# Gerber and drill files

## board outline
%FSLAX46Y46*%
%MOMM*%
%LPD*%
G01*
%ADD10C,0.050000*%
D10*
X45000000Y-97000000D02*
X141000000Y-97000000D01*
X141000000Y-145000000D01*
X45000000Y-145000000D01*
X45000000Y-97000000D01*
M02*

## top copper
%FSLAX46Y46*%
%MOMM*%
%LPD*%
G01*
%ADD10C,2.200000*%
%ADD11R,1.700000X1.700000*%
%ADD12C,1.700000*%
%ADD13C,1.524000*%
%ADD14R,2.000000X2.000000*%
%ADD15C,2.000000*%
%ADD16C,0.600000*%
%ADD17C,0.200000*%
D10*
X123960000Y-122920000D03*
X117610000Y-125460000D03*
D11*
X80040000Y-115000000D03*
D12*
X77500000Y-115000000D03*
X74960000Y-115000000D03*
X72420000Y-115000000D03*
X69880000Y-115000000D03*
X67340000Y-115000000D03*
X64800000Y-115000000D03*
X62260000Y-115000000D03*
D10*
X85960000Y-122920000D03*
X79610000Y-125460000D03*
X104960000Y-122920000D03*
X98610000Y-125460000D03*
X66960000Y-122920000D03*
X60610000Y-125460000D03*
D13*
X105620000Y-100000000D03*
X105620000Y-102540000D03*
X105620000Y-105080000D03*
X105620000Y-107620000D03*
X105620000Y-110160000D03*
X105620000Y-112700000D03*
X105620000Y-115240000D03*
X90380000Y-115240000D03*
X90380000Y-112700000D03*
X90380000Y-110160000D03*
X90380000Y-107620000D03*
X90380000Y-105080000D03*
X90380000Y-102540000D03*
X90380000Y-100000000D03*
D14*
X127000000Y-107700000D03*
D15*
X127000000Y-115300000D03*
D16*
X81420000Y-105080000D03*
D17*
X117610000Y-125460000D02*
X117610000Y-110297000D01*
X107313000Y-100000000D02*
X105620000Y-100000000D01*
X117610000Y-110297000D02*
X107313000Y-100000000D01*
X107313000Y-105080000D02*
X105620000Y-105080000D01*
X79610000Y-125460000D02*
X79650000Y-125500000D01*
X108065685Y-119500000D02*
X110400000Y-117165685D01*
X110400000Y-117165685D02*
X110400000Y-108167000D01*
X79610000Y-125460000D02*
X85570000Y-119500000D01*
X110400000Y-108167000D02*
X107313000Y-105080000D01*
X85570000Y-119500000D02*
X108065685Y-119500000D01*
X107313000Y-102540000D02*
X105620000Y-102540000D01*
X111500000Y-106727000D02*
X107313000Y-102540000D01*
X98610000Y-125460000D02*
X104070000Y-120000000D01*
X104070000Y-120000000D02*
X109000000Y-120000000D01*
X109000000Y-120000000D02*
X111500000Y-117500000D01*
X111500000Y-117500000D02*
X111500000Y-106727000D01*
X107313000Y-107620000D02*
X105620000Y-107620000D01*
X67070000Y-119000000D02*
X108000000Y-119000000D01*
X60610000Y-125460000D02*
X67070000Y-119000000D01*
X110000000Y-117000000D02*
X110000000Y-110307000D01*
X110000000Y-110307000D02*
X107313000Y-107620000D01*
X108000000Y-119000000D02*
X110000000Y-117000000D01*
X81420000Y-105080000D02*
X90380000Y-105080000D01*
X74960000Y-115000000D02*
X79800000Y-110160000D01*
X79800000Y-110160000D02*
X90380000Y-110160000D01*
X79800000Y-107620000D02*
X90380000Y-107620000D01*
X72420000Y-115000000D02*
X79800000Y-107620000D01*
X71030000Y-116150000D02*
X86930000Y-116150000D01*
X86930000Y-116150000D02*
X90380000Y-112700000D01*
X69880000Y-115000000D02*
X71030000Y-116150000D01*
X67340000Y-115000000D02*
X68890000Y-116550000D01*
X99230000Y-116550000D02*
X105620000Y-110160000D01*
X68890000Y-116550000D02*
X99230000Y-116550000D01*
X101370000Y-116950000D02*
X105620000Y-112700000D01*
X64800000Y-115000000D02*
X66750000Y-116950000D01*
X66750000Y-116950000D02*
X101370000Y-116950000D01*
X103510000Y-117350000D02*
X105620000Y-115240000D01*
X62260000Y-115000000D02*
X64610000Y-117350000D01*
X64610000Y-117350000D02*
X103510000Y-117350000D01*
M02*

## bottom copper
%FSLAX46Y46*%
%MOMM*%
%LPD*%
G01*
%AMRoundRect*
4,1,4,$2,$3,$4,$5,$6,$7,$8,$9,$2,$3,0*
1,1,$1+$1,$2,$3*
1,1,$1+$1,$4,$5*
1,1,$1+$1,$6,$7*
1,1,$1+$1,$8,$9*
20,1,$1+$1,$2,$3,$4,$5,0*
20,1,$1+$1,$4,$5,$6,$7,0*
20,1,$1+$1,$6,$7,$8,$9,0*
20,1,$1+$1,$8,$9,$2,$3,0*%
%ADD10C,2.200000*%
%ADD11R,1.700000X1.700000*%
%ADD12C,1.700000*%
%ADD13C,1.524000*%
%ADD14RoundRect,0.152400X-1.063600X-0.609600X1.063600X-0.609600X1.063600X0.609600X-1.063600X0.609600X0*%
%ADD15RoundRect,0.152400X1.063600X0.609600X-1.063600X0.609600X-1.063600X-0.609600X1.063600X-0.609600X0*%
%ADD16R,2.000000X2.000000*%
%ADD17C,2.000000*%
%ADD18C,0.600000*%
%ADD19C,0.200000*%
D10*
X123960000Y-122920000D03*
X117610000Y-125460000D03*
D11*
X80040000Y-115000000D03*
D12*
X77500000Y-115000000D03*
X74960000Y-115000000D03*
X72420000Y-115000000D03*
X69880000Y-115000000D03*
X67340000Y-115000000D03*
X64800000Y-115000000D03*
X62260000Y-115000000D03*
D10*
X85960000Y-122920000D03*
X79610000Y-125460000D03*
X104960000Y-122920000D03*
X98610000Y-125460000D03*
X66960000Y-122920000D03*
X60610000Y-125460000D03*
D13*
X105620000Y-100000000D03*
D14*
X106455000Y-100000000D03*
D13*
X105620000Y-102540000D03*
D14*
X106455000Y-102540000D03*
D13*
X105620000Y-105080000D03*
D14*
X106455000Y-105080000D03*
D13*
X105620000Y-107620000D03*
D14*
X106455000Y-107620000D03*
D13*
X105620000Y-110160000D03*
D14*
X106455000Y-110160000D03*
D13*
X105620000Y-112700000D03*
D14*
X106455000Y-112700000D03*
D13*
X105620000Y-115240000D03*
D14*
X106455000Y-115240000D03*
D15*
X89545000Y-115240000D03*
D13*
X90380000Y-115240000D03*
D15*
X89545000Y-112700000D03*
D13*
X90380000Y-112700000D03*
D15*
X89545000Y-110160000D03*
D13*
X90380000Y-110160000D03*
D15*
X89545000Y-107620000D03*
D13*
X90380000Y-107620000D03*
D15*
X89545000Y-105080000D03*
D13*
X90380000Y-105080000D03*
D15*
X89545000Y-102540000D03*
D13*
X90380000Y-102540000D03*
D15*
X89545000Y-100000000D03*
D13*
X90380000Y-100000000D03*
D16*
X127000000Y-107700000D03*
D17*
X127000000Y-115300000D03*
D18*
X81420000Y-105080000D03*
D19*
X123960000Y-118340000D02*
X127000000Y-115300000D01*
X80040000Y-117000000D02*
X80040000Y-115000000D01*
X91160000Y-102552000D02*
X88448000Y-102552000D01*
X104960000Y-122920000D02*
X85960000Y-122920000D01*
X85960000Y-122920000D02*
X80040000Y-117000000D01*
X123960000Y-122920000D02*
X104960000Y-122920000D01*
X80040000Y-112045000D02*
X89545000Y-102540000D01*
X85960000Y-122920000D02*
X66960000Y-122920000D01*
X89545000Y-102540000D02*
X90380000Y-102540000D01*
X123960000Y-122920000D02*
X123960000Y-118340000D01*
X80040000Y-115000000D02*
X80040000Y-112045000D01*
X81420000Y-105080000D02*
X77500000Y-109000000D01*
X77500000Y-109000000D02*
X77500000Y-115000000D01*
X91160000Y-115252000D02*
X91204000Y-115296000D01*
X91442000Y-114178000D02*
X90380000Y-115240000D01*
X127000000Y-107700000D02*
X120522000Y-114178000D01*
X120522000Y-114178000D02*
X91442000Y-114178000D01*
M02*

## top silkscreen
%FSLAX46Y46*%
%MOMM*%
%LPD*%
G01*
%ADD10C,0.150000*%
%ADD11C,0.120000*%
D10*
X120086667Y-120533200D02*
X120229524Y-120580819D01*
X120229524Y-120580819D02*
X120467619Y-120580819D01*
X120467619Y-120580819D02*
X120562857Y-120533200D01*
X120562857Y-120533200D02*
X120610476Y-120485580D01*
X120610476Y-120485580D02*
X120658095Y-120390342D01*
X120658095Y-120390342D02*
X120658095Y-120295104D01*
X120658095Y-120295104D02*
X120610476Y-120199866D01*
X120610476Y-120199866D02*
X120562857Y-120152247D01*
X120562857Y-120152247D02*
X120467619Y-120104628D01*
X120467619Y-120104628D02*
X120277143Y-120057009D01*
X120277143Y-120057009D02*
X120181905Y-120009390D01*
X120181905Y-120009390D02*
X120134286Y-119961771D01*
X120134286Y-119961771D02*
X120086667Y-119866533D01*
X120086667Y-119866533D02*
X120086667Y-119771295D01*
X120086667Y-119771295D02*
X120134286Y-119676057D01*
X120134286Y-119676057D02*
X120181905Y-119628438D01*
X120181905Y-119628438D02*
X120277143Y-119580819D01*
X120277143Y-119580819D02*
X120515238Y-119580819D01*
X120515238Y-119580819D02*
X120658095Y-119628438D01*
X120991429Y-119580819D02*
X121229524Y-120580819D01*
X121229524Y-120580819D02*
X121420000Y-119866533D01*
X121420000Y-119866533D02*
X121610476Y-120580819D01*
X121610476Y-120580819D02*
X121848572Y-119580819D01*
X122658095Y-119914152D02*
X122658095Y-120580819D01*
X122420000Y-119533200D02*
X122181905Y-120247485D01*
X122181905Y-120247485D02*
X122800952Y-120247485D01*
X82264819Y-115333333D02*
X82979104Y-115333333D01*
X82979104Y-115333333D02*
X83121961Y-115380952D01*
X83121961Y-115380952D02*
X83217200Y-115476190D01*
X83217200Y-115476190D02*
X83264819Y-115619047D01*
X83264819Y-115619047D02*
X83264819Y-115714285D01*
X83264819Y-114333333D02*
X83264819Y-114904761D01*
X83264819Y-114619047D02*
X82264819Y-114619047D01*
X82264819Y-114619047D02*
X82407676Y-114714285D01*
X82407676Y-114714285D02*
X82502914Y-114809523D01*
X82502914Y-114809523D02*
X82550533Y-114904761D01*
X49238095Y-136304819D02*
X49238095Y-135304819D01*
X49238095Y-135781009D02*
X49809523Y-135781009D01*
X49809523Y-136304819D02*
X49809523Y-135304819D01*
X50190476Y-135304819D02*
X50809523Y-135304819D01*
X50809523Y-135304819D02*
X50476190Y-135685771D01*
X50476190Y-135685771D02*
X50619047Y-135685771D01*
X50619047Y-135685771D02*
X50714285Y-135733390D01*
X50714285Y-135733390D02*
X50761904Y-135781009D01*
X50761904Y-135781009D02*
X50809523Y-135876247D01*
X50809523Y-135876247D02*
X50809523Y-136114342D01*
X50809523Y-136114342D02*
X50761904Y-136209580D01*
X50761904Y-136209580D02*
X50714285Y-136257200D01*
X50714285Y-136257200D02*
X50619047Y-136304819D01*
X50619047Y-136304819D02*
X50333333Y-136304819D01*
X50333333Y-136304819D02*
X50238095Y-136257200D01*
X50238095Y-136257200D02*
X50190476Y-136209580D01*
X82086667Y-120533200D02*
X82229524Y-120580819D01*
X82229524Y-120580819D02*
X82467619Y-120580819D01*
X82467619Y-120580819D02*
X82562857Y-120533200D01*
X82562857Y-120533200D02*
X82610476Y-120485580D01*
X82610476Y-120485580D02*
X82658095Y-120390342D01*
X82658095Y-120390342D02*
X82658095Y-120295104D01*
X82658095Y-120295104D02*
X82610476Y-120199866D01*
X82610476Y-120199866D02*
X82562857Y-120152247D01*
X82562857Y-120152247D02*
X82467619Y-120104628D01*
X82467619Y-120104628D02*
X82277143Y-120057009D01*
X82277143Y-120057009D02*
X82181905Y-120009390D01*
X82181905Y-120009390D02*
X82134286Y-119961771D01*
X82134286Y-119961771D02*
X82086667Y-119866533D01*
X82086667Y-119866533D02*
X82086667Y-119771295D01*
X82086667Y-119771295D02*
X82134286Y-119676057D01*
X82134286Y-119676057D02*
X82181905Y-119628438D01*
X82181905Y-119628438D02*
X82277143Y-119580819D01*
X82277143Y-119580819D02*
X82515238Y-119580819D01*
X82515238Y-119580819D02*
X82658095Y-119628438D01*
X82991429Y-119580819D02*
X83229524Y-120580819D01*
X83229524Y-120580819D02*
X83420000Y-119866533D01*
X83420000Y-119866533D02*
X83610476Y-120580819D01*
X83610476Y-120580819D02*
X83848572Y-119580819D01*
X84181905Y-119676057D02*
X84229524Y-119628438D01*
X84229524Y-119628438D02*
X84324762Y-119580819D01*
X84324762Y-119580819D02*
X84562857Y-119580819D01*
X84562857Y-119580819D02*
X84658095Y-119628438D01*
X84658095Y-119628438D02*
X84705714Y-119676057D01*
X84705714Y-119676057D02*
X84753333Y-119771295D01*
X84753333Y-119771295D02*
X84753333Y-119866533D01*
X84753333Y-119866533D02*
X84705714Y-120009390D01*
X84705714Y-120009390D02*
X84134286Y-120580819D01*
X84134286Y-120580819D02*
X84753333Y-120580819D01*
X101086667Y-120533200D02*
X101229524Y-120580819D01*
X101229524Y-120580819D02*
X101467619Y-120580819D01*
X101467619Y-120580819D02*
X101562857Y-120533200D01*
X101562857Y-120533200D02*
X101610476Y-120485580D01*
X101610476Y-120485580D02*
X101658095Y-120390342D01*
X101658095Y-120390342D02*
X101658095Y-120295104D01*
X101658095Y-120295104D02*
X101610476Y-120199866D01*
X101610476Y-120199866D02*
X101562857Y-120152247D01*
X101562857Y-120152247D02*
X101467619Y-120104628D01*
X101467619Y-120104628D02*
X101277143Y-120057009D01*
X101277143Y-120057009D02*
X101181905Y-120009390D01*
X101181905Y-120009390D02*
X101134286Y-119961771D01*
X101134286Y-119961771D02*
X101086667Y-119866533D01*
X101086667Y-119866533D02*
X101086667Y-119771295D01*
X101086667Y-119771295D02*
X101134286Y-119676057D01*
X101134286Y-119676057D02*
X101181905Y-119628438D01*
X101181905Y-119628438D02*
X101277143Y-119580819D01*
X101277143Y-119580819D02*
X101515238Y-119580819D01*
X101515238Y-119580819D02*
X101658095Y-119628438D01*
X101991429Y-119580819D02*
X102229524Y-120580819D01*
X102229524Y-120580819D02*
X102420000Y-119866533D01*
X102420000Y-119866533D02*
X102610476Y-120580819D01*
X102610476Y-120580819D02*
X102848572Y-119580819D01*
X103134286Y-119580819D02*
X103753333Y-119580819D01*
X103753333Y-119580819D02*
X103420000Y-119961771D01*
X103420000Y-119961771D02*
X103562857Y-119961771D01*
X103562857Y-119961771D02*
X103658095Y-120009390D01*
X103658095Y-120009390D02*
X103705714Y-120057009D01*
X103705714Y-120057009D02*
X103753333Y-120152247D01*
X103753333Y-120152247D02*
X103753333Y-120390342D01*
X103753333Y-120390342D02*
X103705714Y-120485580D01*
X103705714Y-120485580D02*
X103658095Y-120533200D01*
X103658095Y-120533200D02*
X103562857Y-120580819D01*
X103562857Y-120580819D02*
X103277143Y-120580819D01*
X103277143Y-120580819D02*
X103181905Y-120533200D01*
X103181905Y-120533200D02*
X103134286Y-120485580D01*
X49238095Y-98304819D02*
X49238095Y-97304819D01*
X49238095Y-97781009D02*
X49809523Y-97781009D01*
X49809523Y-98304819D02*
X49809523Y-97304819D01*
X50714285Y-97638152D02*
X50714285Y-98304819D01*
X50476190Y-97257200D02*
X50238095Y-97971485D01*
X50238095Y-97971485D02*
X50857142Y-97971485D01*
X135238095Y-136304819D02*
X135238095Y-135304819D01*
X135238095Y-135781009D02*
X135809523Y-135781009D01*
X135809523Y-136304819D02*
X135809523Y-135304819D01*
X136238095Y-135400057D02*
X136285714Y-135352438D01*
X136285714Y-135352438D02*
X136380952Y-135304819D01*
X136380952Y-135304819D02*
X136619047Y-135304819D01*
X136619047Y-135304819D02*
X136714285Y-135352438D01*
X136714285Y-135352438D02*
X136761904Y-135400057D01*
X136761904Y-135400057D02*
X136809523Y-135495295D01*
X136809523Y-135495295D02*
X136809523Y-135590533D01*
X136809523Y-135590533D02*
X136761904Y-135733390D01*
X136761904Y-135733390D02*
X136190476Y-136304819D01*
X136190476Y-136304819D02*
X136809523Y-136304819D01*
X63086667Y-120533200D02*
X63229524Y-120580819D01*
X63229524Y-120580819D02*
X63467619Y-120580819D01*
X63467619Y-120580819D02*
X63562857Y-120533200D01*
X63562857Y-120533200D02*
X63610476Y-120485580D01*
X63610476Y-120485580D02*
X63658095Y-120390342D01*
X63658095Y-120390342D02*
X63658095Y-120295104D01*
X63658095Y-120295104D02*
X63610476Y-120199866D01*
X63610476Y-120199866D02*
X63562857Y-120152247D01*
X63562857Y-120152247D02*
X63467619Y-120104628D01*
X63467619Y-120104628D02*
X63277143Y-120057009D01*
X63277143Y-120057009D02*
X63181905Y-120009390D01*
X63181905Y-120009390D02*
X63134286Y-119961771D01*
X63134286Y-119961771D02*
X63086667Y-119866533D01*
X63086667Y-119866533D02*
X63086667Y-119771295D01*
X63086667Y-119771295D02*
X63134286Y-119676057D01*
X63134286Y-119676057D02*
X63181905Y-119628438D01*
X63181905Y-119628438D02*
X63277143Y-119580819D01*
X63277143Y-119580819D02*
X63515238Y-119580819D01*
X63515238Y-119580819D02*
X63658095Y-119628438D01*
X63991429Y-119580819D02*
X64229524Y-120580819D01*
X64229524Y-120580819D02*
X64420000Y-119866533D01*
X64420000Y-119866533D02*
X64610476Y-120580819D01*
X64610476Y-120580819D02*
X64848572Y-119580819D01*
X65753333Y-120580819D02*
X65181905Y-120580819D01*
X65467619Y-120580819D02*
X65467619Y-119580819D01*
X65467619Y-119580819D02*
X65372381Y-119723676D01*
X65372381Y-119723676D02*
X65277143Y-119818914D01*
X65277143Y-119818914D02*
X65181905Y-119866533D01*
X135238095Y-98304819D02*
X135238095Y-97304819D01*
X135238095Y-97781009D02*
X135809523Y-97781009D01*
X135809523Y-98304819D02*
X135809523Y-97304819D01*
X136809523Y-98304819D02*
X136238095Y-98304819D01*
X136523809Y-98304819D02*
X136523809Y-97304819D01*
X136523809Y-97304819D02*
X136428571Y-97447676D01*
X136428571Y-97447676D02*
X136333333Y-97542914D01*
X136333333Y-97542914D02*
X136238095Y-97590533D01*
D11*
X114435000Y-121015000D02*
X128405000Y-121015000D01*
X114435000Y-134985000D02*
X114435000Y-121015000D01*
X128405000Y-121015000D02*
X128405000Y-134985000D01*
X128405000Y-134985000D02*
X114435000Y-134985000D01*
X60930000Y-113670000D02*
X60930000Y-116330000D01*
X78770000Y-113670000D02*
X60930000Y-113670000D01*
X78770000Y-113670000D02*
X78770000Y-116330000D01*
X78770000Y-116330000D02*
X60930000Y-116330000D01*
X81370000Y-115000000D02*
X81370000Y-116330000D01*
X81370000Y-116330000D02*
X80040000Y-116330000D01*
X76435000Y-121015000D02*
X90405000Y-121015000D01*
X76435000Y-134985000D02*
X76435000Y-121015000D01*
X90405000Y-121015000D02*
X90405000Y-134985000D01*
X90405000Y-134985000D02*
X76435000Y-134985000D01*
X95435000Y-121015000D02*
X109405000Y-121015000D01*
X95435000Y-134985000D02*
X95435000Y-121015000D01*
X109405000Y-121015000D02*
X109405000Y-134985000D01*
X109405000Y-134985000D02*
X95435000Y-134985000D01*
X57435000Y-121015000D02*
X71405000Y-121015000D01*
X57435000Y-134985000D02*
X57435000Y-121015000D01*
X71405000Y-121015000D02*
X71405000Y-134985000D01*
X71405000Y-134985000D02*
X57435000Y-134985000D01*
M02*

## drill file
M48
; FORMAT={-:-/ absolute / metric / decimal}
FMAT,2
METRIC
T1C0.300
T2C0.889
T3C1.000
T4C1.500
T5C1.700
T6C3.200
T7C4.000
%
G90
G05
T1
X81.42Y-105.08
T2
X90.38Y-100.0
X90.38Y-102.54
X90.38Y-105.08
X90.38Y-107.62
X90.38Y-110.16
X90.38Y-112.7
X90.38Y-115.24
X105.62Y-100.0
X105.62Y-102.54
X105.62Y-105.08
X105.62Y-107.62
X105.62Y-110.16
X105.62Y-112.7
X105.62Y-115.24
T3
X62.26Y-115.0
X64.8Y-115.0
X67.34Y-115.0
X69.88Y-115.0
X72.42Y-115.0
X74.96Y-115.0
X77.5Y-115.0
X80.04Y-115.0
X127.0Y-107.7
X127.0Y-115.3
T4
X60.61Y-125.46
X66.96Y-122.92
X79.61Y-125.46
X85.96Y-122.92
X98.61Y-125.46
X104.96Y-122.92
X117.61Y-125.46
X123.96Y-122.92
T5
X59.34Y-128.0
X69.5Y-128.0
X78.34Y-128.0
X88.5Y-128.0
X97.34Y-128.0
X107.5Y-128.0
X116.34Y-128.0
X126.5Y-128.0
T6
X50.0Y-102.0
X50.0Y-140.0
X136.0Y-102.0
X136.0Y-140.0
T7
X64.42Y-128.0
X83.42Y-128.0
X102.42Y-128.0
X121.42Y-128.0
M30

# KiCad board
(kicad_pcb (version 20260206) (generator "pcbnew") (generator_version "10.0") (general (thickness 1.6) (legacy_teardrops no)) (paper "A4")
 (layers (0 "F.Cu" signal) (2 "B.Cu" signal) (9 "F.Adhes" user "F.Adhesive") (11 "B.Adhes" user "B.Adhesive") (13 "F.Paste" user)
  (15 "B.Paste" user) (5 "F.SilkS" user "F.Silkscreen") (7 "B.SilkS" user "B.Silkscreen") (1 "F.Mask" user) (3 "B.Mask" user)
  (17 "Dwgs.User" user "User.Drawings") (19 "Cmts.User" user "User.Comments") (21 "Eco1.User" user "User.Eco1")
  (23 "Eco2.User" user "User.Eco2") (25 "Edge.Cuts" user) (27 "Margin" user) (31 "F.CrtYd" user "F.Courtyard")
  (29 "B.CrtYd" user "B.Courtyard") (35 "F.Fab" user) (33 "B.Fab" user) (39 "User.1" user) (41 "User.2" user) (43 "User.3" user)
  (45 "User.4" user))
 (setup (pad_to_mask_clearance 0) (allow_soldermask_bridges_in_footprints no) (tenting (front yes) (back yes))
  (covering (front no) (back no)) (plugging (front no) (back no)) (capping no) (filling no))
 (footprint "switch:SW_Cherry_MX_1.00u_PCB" (layer "F.Cu") (at 123.96 122.92)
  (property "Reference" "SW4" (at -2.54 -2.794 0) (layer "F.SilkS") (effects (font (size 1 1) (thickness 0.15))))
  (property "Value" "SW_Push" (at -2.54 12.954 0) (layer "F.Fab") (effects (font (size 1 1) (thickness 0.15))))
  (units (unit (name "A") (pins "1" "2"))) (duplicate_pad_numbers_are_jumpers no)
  (fp_line (start -9.525 -1.905) (end 4.445 -1.905) (stroke (width 0.12) (type solid)) (layer "F.SilkS"))
  (fp_line (start -9.525 12.065) (end -9.525 -1.905) (stroke (width 0.12) (type solid)) (layer "F.SilkS"))
  (fp_line (start 4.445 -1.905) (end 4.445 12.065) (stroke (width 0.12) (type solid)) (layer "F.SilkS"))
  (fp_line (start 4.445 12.065) (end -9.525 12.065) (stroke (width 0.12) (type solid)) (layer "F.SilkS"))
  (pad "" np_thru_hole circle (at -7.62 5.08) (size 1.7 1.7) (drill 1.7) (layers "*.Cu" "*.Mask"))
  (pad "" np_thru_hole circle (at -2.54 5.08) (size 4 4) (drill 4) (layers "*.Cu" "*.Mask"))
  (pad "" np_thru_hole circle (at 2.54 5.08) (size 1.7 1.7) (drill 1.7) (layers "*.Cu" "*.Mask"))
  (pad "1" thru_hole circle (at 0 0) (size 2.2 2.2) (drill 1.5) (layers "*.Cu" "*.Mask") (remove_unused_layers no) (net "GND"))
  (pad "2" thru_hole circle (at -6.35 2.54) (size 2.2 2.2) (drill 1.5) (layers "*.Cu" "*.Mask") (remove_unused_layers no)
   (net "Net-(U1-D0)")))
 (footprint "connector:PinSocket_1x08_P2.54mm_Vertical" (layer "F.Cu") (at 80.04 115 -90)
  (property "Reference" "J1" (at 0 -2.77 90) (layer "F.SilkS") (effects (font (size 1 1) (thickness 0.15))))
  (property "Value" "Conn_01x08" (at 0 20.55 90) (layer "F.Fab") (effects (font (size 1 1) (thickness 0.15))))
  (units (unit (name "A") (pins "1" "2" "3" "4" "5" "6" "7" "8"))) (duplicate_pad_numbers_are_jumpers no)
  (fp_line (start -1.33 19.11) (end 1.33 19.11) (stroke (width 0.12) (type solid)) (layer "F.SilkS"))
  (fp_line (start -1.33 1.27) (end -1.33 19.11) (stroke (width 0.12) (type solid)) (layer "F.SilkS"))
  (fp_line (start -1.33 1.27) (end 1.33 1.27) (stroke (width 0.12) (type solid)) (layer "F.SilkS"))
  (fp_line (start 1.33 1.27) (end 1.33 19.11) (stroke (width 0.12) (type solid)) (layer "F.SilkS"))
  (fp_line (start 0 -1.33) (end 1.33 -1.33) (stroke (width 0.12) (type solid)) (layer "F.SilkS"))
  (fp_line (start 1.33 -1.33) (end 1.33 0) (stroke (width 0.12) (type solid)) (layer "F.SilkS"))
  (pad "1" thru_hole rect (at 0 0 270) (size 1.7 1.7) (drill 1) (layers "*.Cu" "*.Mask") (remove_unused_layers no) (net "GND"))
  (pad "2" thru_hole circle (at 0 2.54 270) (size 1.7 1.7) (drill 1) (layers "*.Cu" "*.Mask") (remove_unused_layers no) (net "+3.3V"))
  (pad "3" thru_hole circle (at 0 5.08 270) (size 1.7 1.7) (drill 1) (layers "*.Cu" "*.Mask") (remove_unused_layers no) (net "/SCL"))
  (pad "4" thru_hole circle (at 0 7.62 270) (size 1.7 1.7) (drill 1) (layers "*.Cu" "*.Mask") (remove_unused_layers no) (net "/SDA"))
  (pad "5" thru_hole circle (at 0 10.16 270) (size 1.7 1.7) (drill 1) (layers "*.Cu" "*.Mask") (remove_unused_layers no) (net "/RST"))
  (pad "6" thru_hole circle (at 0 12.7 270) (size 1.7 1.7) (drill 1) (layers "*.Cu" "*.Mask") (remove_unused_layers no) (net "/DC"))
  (pad "7" thru_hole circle (at 0 15.24 270) (size 1.7 1.7) (drill 1) (layers "*.Cu" "*.Mask") (remove_unused_layers no) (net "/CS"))
  (pad "8" thru_hole circle (at 0 17.78 270) (size 1.7 1.7) (drill 1) (layers "*.Cu" "*.Mask") (remove_unused_layers no) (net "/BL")))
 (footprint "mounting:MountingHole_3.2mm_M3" (layer "F.Cu") (at 50 140)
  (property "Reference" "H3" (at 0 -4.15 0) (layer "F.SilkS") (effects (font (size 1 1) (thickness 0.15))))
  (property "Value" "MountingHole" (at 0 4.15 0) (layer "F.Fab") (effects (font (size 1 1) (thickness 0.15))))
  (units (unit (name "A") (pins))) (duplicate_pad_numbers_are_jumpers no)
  (pad "" np_thru_hole circle (at 0 0) (size 3.2 3.2) (drill 3.2) (layers "*.Cu" "*.Mask")))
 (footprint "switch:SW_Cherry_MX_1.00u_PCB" (layer "F.Cu") (at 85.96 122.92)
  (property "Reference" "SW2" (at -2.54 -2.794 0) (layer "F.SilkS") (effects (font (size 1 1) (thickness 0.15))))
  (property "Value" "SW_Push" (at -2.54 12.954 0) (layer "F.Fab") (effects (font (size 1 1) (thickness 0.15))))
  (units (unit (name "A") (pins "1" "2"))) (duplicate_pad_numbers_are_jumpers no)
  (fp_line (start -9.525 -1.905) (end 4.445 -1.905) (stroke (width 0.12) (type solid)) (layer "F.SilkS"))
  (fp_line (start -9.525 12.065) (end -9.525 -1.905) (stroke (width 0.12) (type solid)) (layer "F.SilkS"))
  (fp_line (start 4.445 -1.905) (end 4.445 12.065) (stroke (width 0.12) (type solid)) (layer "F.SilkS"))
  (fp_line (start 4.445 12.065) (end -9.525 12.065) (stroke (width 0.12) (type solid)) (layer "F.SilkS"))
  (pad "" np_thru_hole circle (at -7.62 5.08) (size 1.7 1.7) (drill 1.7) (layers "*.Cu" "*.Mask"))
  (pad "" np_thru_hole circle (at -2.54 5.08) (size 4 4) (drill 4) (layers "*.Cu" "*.Mask"))
  (pad "" np_thru_hole circle (at 2.54 5.08) (size 1.7 1.7) (drill 1.7) (layers "*.Cu" "*.Mask"))
  (pad "1" thru_hole circle (at 0 0) (size 2.2 2.2) (drill 1.5) (layers "*.Cu" "*.Mask") (remove_unused_layers no) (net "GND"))
  (pad "2" thru_hole circle (at -6.35 2.54) (size 2.2 2.2) (drill 1.5) (layers "*.Cu" "*.Mask") (remove_unused_layers no)
   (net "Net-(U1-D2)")))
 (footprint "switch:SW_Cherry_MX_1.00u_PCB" (layer "F.Cu") (at 104.96 122.92)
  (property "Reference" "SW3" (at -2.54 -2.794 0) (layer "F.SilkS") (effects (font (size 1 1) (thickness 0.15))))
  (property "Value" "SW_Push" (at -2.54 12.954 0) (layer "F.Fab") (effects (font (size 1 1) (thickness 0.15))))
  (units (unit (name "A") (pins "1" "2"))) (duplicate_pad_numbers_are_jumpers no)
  (fp_line (start -9.525 -1.905) (end 4.445 -1.905) (stroke (width 0.12) (type solid)) (layer "F.SilkS"))
  (fp_line (start -9.525 12.065) (end -9.525 -1.905) (stroke (width 0.12) (type solid)) (layer "F.SilkS"))
  (fp_line (start 4.445 -1.905) (end 4.445 12.065) (stroke (width 0.12) (type solid)) (layer "F.SilkS"))
  (fp_line (start 4.445 12.065) (end -9.525 12.065) (stroke (width 0.12) (type solid)) (layer "F.SilkS"))
  (pad "" np_thru_hole circle (at -7.62 5.08) (size 1.7 1.7) (drill 1.7) (layers "*.Cu" "*.Mask"))
  (pad "" np_thru_hole circle (at -2.54 5.08) (size 4 4) (drill 4) (layers "*.Cu" "*.Mask"))
  (pad "" np_thru_hole circle (at 2.54 5.08) (size 1.7 1.7) (drill 1.7) (layers "*.Cu" "*.Mask"))
  (pad "1" thru_hole circle (at 0 0) (size 2.2 2.2) (drill 1.5) (layers "*.Cu" "*.Mask") (remove_unused_layers no) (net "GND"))
  (pad "2" thru_hole circle (at -6.35 2.54) (size 2.2 2.2) (drill 1.5) (layers "*.Cu" "*.Mask") (remove_unused_layers no)
   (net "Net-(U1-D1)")))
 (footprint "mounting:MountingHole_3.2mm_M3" (layer "F.Cu") (at 50 102)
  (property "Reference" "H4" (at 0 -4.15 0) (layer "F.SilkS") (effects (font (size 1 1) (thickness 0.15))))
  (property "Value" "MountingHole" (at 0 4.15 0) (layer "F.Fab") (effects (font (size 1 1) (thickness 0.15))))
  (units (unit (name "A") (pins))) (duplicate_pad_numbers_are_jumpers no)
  (pad "" np_thru_hole circle (at 0 0) (size 3.2 3.2) (drill 3.2) (layers "*.Cu" "*.Mask")))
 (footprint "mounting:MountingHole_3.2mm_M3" (layer "F.Cu") (at 136 140)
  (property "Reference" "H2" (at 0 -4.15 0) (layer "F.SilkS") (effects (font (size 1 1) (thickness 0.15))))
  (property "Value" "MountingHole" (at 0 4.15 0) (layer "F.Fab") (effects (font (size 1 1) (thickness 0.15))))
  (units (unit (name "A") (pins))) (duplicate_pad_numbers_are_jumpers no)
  (pad "" np_thru_hole circle (at 0 0) (size 3.2 3.2) (drill 3.2) (layers "*.Cu" "*.Mask")))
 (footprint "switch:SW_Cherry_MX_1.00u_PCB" (layer "F.Cu") (at 66.96 122.92)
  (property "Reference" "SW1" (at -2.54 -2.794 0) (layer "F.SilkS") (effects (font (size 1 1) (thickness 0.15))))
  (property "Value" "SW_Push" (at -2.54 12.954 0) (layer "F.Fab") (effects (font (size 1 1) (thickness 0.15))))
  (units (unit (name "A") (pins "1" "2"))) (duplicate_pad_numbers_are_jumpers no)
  (fp_line (start -9.525 -1.905) (end 4.445 -1.905) (stroke (width 0.12) (type solid)) (layer "F.SilkS"))
  (fp_line (start -9.525 12.065) (end -9.525 -1.905) (stroke (width 0.12) (type solid)) (layer "F.SilkS"))
  (fp_line (start 4.445 -1.905) (end 4.445 12.065) (stroke (width 0.12) (type solid)) (layer "F.SilkS"))
  (fp_line (start 4.445 12.065) (end -9.525 12.065) (stroke (width 0.12) (type solid)) (layer "F.SilkS"))
  (pad "" np_thru_hole circle (at -7.62 5.08) (size 1.7 1.7) (drill 1.7) (layers "*.Cu" "*.Mask"))
  (pad "" np_thru_hole circle (at -2.54 5.08) (size 4 4) (drill 4) (layers "*.Cu" "*.Mask"))
  (pad "" np_thru_hole circle (at 2.54 5.08) (size 1.7 1.7) (drill 1.7) (layers "*.Cu" "*.Mask"))
  (pad "1" thru_hole circle (at 0 0) (size 2.2 2.2) (drill 1.5) (layers "*.Cu" "*.Mask") (remove_unused_layers no) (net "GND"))
  (pad "2" thru_hole circle (at -6.35 2.54) (size 2.2 2.2) (drill 1.5) (layers "*.Cu" "*.Mask") (remove_unused_layers no)
   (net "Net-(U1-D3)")))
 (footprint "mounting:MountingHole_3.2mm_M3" (layer "F.Cu") (at 136 102)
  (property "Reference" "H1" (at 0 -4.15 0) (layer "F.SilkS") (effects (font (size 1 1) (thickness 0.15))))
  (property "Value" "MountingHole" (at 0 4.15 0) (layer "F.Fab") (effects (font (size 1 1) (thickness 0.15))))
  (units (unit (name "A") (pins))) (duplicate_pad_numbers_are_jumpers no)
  (pad "" np_thru_hole circle (at 0 0) (size 3.2 3.2) (drill 3.2) (layers "*.Cu" "*.Mask")))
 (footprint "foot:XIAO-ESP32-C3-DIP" (layer "B.Cu") (at 98 107.62 90)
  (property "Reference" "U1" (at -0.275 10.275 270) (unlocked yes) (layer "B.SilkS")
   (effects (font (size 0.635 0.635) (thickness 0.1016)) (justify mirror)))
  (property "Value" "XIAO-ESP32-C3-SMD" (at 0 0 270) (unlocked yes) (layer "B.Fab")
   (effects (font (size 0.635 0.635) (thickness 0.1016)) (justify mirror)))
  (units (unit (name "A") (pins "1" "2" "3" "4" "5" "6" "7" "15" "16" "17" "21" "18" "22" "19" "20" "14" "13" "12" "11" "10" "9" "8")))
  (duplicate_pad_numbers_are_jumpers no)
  (pad "1" thru_hole circle (at 7.62 7.62) (size 1.524 1.524) (drill 0.889) (layers "*.Cu" "*.Mask") (remove_unused_layers no)
   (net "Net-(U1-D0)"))
  (pad "1" smd roundrect (at 7.62 8.455) (size 2.432 1.524) (layers "B.Cu" "B.Mask") (roundrect_rratio 0.1) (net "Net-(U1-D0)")
   (thermal_bridge_angle 45))
  (pad "2" thru_hole circle (at 5.08 7.62) (size 1.524 1.524) (drill 0.889) (layers "*.Cu" "*.Mask") (remove_unused_layers no)
   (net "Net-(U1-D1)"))
  (pad "2" smd roundrect (at 5.08 8.455) (size 2.432 1.524) (layers "B.Cu" "B.Mask") (roundrect_rratio 0.1) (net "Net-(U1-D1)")
   (thermal_bridge_angle 45))
  (pad "3" thru_hole circle (at 2.54 7.62) (size 1.524 1.524) (drill 0.889) (layers "*.Cu" "*.Mask") (remove_unused_layers no)
   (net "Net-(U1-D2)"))
  (pad "3" smd roundrect (at 2.54 8.455) (size 2.432 1.524) (layers "B.Cu" "B.Mask") (roundrect_rratio 0.1) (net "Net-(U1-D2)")
   (thermal_bridge_angle 45))
  (pad "4" thru_hole circle (at 0 7.62) (size 1.524 1.524) (drill 0.889) (layers "*.Cu" "*.Mask") (remove_unused_layers no)
   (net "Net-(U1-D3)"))
  (pad "4" smd roundrect (at 0 8.455) (size 2.432 1.524) (layers "B.Cu" "B.Mask") (roundrect_rratio 0.1) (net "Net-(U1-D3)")
   (thermal_bridge_angle 45))
  (pad "5" thru_hole circle (at -2.54 7.62) (size 1.524 1.524) (drill 0.889) (layers "*.Cu" "*.Mask") (remove_unused_layers no) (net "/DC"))
  (pad "5" smd roundrect (at -2.54 8.455) (size 2.432 1.524) (layers "B.Cu" "B.Mask") (roundrect_rratio 0.1) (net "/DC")
   (thermal_bridge_angle 45))
  (pad "6" thru_hole circle (at -5.08 7.62) (size 1.524 1.524) (drill 0.889) (layers "*.Cu" "*.Mask") (remove_unused_layers no) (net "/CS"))
  (pad "6" smd roundrect (at -5.08 8.455) (size 2.432 1.524) (layers "B.Cu" "B.Mask") (roundrect_rratio 0.1) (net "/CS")
   (thermal_bridge_angle 45))
  (pad "7" thru_hole circle (at -7.62 7.62) (size 1.524 1.524) (drill 0.889) (layers "*.Cu" "*.Mask") (remove_unused_layers no) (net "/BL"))
  (pad "7" smd roundrect (at -7.62 8.455) (size 2.432 1.524) (layers "B.Cu" "B.Mask") (roundrect_rratio 0.1) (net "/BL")
   (thermal_bridge_angle 45))
  (pad "8" smd roundrect (at -7.62 -8.455 180) (size 2.432 1.524) (layers "B.Cu" "B.Mask") (roundrect_rratio 0.1) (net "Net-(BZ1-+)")
   (thermal_bridge_angle 45))
  (pad "8" thru_hole circle (at -7.62 -7.62 180) (size 1.524 1.524) (drill 0.889) (layers "*.Cu" "*.Mask") (remove_unused_layers no)
   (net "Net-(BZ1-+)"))
  (pad "9" smd roundrect (at -5.08 -8.455 180) (size 2.432 1.524) (layers "B.Cu" "B.Mask") (roundrect_rratio 0.1) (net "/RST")
   (thermal_bridge_angle 45))
  (pad "9" thru_hole circle (at -5.08 -7.62 180) (size 1.524 1.524) (drill 0.889) (layers "*.Cu" "*.Mask") (remove_unused_layers no)
   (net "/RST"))
  (pad "10" smd roundrect (at -2.54 -8.455 180) (size 2.432 1.524) (layers "B.Cu" "B.Mask") (roundrect_rratio 0.1) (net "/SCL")
   (thermal_bridge_angle 45))
  (pad "10" thru_hole circle (at -2.54 -7.62 180) (size 1.524 1.524) (drill 0.889) (layers "*.Cu" "*.Mask") (remove_unused_layers no)
   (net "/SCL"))
  (pad "11" smd roundrect (at 0 -8.455 180) (size 2.432 1.524) (layers "B.Cu" "B.Mask") (roundrect_rratio 0.1) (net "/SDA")
   (thermal_bridge_angle 45))
  (pad "11" thru_hole circle (at 0 -7.62 180) (size 1.524 1.524) (drill 0.889) (layers "*.Cu" "*.Mask") (remove_unused_layers no)
   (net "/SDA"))
  (pad "12" smd roundrect (at 2.54 -8.455 180) (size 2.432 1.524) (layers "B.Cu" "B.Mask") (roundrect_rratio 0.1) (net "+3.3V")
   (thermal_bridge_angle 45))
  (pad "12" thru_hole circle (at 2.54 -7.62 180) (size 1.524 1.524) (drill 0.889) (layers "*.Cu" "*.Mask") (remove_unused_layers no)
   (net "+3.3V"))
  (pad "13" smd roundrect (at 5.08 -8.455 180) (size 2.432 1.524) (layers "B.Cu" "B.Mask") (roundrect_rratio 0.1) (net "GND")
   (thermal_bridge_angle 45))
  (pad "13" thru_hole circle (at 5.08 -7.62 180) (size 1.524 1.524) (drill 0.889) (layers "*.Cu" "*.Mask") (remove_unused_layers no)
   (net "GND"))
  (pad "14" smd roundrect (at 7.62 -8.455 180) (size 2.432 1.524) (layers "B.Cu" "B.Mask") (roundrect_rratio 0.1)
   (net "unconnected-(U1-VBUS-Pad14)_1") (thermal_bridge_angle 45))
  (pad "14" thru_hole circle (at 7.62 -7.62 180) (size 1.524 1.524) (drill 0.889) (layers "*.Cu" "*.Mask") (remove_unused_layers no)
   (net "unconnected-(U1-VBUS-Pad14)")))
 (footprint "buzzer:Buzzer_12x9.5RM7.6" (layer "B.Cu") (at 127 107.7 -90)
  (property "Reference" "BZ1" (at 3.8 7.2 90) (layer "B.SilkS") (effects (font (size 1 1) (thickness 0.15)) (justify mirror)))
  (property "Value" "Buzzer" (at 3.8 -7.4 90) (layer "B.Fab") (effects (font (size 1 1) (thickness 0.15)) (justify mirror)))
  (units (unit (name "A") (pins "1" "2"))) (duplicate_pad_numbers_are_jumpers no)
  (pad "1" thru_hole rect (at 0 0 270) (size 2 2) (drill 1) (layers "*.Cu" "*.Mask") (remove_unused_layers no) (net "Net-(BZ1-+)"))
  (pad "2" thru_hole circle (at 7.6 0 270) (size 2 2) (drill 1) (layers "*.Cu" "*.Mask") (remove_unused_layers no) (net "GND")))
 (gr_rect (start 45 97) (end 141 145) (stroke (width 0.05) (type default)) (fill no) (layer "Edge.Cuts"))
 (segment (start 123.96 118.34) (end 127 115.3) (width 0.2) (layer "B.Cu") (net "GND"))
 (segment (start 80.04 117) (end 80.04 115) (width 0.2) (layer "B.Cu") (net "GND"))
 (segment (start 91.16 102.552) (end 88.448 102.552) (width 0.2) (layer "B.Cu") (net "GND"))
 (segment (start 104.96 122.92) (end 85.96 122.92) (width 0.2) (layer "B.Cu") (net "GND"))
 (segment (start 85.96 122.92) (end 80.04 117) (width 0.2) (layer "B.Cu") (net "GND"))
 (segment (start 123.96 122.92) (end 104.96 122.92) (width 0.2) (layer "B.Cu") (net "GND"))
 (segment (start 80.04 112.045) (end 89.545 102.54) (width 0.2) (layer "B.Cu") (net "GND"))
 (segment (start 85.96 122.92) (end 66.96 122.92) (width 0.2) (layer "B.Cu") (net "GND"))
 (segment (start 89.545 102.54) (end 90.38 102.54) (width 0.2) (layer "B.Cu") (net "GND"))
 (segment (start 123.96 122.92) (end 123.96 118.34) (width 0.2) (layer "B.Cu") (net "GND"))
 (segment (start 80.04 115) (end 80.04 112.045) (width 0.2) (layer "B.Cu") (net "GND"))
 (segment (start 117.61 125.46) (end 117.61 110.297) (width 0.2) (layer "F.Cu") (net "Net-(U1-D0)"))
 (segment (start 107.313 100) (end 105.62 100) (width 0.2) (layer "F.Cu") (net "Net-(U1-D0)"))
 (segment (start 117.61 110.297) (end 107.313 100) (width 0.2) (layer "F.Cu") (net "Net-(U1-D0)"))
 (segment (start 107.313 105.08) (end 105.62 105.08) (width 0.2) (layer "F.Cu") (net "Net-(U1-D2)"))
 (segment (start 79.61 125.46) (end 79.65 125.5) (width 0.2) (layer "F.Cu") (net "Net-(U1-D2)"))
 (segment (start 108.065685 119.5) (end 110.4 117.165685) (width 0.2) (layer "F.Cu") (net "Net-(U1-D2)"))
 (segment (start 110.4 117.165685) (end 110.4 108.167) (width 0.2) (layer "F.Cu") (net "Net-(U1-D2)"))
 (segment (start 79.61 125.46) (end 85.57 119.5) (width 0.2) (layer "F.Cu") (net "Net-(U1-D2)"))
 (segment (start 110.4 108.167) (end 107.313 105.08) (width 0.2) (layer "F.Cu") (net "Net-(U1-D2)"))
 (segment (start 85.57 119.5) (end 108.065685 119.5) (width 0.2) (layer "F.Cu") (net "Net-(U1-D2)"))
 (segment (start 107.313 102.54) (end 105.62 102.54) (width 0.2) (layer "F.Cu") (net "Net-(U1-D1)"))
 (segment (start 111.5 106.727) (end 107.313 102.54) (width 0.2) (layer "F.Cu") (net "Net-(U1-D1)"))
 (segment (start 98.61 125.46) (end 104.07 120) (width 0.2) (layer "F.Cu") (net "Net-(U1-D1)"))
 (segment (start 104.07 120) (end 109 120) (width 0.2) (layer "F.Cu") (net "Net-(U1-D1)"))
 (segment (start 109 120) (end 111.5 117.5) (width 0.2) (layer "F.Cu") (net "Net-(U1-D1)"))
 (segment (start 111.5 117.5) (end 111.5 106.727) (width 0.2) (layer "F.Cu") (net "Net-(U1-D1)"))
 (segment (start 107.313 107.62) (end 105.62 107.62) (width 0.2) (layer "F.Cu") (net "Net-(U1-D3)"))
 (segment (start 67.07 119) (end 108 119) (width 0.2) (layer "F.Cu") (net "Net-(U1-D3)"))
 (segment (start 60.61 125.46) (end 67.07 119) (width 0.2) (layer "F.Cu") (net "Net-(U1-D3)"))
 (segment (start 110 117) (end 110 110.307) (width 0.2) (layer "F.Cu") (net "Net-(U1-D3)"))
 (segment (start 110 110.307) (end 107.313 107.62) (width 0.2) (layer "F.Cu") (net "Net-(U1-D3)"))
 (segment (start 108 119) (end 110 117) (width 0.2) (layer "F.Cu") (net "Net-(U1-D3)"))
 (segment (start 81.42 105.08) (end 90.38 105.08) (width 0.2) (layer "F.Cu") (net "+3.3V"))
 (via (at 81.42 105.08) (size 0.6) (drill 0.3) (layers "F.Cu" "B.Cu") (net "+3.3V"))
 (segment (start 81.42 105.08) (end 77.5 109) (width 0.2) (layer "B.Cu") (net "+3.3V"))
 (segment (start 77.5 109) (end 77.5 115) (width 0.2) (layer "B.Cu") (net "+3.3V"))
 (segment (start 74.96 115) (end 79.8 110.16) (width 0.2) (layer "F.Cu") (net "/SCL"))
 (segment (start 79.8 110.16) (end 90.38 110.16) (width 0.2) (layer "F.Cu") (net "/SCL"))
 (segment (start 79.8 107.62) (end 90.38 107.62) (width 0.2) (layer "F.Cu") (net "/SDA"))
 (segment (start 72.42 115) (end 79.8 107.62) (width 0.2) (layer "F.Cu") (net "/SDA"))
 (segment (start 71.03 116.15) (end 86.93 116.15) (width 0.2) (layer "F.Cu") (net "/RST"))
 (segment (start 86.93 116.15) (end 90.38 112.7) (width 0.2) (layer "F.Cu") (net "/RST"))
 (segment (start 69.88 115) (end 71.03 116.15) (width 0.2) (layer "F.Cu") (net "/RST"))
 (segment (start 67.34 115) (end 68.89 116.55) (width 0.2) (layer "F.Cu") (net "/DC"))
 (segment (start 99.23 116.55) (end 105.62 110.16) (width 0.2) (layer "F.Cu") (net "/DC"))
 (segment (start 68.89 116.55) (end 99.23 116.55) (width 0.2) (layer "F.Cu") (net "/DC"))
 (segment (start 101.37 116.95) (end 105.62 112.7) (width 0.2) (layer "F.Cu") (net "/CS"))
 (segment (start 64.8 115) (end 66.75 116.95) (width 0.2) (layer "F.Cu") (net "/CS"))
 (segment (start 66.75 116.95) (end 101.37 116.95) (width 0.2) (layer "F.Cu") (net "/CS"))
 (segment (start 103.51 117.35) (end 105.62 115.24) (width 0.2) (layer "F.Cu") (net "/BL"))
 (segment (start 62.26 115) (end 64.61 117.35) (width 0.2) (layer "F.Cu") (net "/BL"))
 (segment (start 64.61 117.35) (end 103.51 117.35) (width 0.2) (layer "F.Cu") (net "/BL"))
 (segment (start 91.16 115.252) (end 91.204 115.296) (width 0.2) (layer "B.Cu") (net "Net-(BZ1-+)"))
 (segment (start 91.442 114.178) (end 90.38 115.24) (width 0.2) (layer "B.Cu") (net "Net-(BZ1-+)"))
 (segment (start 127 107.7) (end 120.522 114.178) (width 0.2) (layer "B.Cu") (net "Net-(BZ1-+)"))
 (segment (start 120.522 114.178) (end 91.442 114.178) (width 0.2) (layer "B.Cu") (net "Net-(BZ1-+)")))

